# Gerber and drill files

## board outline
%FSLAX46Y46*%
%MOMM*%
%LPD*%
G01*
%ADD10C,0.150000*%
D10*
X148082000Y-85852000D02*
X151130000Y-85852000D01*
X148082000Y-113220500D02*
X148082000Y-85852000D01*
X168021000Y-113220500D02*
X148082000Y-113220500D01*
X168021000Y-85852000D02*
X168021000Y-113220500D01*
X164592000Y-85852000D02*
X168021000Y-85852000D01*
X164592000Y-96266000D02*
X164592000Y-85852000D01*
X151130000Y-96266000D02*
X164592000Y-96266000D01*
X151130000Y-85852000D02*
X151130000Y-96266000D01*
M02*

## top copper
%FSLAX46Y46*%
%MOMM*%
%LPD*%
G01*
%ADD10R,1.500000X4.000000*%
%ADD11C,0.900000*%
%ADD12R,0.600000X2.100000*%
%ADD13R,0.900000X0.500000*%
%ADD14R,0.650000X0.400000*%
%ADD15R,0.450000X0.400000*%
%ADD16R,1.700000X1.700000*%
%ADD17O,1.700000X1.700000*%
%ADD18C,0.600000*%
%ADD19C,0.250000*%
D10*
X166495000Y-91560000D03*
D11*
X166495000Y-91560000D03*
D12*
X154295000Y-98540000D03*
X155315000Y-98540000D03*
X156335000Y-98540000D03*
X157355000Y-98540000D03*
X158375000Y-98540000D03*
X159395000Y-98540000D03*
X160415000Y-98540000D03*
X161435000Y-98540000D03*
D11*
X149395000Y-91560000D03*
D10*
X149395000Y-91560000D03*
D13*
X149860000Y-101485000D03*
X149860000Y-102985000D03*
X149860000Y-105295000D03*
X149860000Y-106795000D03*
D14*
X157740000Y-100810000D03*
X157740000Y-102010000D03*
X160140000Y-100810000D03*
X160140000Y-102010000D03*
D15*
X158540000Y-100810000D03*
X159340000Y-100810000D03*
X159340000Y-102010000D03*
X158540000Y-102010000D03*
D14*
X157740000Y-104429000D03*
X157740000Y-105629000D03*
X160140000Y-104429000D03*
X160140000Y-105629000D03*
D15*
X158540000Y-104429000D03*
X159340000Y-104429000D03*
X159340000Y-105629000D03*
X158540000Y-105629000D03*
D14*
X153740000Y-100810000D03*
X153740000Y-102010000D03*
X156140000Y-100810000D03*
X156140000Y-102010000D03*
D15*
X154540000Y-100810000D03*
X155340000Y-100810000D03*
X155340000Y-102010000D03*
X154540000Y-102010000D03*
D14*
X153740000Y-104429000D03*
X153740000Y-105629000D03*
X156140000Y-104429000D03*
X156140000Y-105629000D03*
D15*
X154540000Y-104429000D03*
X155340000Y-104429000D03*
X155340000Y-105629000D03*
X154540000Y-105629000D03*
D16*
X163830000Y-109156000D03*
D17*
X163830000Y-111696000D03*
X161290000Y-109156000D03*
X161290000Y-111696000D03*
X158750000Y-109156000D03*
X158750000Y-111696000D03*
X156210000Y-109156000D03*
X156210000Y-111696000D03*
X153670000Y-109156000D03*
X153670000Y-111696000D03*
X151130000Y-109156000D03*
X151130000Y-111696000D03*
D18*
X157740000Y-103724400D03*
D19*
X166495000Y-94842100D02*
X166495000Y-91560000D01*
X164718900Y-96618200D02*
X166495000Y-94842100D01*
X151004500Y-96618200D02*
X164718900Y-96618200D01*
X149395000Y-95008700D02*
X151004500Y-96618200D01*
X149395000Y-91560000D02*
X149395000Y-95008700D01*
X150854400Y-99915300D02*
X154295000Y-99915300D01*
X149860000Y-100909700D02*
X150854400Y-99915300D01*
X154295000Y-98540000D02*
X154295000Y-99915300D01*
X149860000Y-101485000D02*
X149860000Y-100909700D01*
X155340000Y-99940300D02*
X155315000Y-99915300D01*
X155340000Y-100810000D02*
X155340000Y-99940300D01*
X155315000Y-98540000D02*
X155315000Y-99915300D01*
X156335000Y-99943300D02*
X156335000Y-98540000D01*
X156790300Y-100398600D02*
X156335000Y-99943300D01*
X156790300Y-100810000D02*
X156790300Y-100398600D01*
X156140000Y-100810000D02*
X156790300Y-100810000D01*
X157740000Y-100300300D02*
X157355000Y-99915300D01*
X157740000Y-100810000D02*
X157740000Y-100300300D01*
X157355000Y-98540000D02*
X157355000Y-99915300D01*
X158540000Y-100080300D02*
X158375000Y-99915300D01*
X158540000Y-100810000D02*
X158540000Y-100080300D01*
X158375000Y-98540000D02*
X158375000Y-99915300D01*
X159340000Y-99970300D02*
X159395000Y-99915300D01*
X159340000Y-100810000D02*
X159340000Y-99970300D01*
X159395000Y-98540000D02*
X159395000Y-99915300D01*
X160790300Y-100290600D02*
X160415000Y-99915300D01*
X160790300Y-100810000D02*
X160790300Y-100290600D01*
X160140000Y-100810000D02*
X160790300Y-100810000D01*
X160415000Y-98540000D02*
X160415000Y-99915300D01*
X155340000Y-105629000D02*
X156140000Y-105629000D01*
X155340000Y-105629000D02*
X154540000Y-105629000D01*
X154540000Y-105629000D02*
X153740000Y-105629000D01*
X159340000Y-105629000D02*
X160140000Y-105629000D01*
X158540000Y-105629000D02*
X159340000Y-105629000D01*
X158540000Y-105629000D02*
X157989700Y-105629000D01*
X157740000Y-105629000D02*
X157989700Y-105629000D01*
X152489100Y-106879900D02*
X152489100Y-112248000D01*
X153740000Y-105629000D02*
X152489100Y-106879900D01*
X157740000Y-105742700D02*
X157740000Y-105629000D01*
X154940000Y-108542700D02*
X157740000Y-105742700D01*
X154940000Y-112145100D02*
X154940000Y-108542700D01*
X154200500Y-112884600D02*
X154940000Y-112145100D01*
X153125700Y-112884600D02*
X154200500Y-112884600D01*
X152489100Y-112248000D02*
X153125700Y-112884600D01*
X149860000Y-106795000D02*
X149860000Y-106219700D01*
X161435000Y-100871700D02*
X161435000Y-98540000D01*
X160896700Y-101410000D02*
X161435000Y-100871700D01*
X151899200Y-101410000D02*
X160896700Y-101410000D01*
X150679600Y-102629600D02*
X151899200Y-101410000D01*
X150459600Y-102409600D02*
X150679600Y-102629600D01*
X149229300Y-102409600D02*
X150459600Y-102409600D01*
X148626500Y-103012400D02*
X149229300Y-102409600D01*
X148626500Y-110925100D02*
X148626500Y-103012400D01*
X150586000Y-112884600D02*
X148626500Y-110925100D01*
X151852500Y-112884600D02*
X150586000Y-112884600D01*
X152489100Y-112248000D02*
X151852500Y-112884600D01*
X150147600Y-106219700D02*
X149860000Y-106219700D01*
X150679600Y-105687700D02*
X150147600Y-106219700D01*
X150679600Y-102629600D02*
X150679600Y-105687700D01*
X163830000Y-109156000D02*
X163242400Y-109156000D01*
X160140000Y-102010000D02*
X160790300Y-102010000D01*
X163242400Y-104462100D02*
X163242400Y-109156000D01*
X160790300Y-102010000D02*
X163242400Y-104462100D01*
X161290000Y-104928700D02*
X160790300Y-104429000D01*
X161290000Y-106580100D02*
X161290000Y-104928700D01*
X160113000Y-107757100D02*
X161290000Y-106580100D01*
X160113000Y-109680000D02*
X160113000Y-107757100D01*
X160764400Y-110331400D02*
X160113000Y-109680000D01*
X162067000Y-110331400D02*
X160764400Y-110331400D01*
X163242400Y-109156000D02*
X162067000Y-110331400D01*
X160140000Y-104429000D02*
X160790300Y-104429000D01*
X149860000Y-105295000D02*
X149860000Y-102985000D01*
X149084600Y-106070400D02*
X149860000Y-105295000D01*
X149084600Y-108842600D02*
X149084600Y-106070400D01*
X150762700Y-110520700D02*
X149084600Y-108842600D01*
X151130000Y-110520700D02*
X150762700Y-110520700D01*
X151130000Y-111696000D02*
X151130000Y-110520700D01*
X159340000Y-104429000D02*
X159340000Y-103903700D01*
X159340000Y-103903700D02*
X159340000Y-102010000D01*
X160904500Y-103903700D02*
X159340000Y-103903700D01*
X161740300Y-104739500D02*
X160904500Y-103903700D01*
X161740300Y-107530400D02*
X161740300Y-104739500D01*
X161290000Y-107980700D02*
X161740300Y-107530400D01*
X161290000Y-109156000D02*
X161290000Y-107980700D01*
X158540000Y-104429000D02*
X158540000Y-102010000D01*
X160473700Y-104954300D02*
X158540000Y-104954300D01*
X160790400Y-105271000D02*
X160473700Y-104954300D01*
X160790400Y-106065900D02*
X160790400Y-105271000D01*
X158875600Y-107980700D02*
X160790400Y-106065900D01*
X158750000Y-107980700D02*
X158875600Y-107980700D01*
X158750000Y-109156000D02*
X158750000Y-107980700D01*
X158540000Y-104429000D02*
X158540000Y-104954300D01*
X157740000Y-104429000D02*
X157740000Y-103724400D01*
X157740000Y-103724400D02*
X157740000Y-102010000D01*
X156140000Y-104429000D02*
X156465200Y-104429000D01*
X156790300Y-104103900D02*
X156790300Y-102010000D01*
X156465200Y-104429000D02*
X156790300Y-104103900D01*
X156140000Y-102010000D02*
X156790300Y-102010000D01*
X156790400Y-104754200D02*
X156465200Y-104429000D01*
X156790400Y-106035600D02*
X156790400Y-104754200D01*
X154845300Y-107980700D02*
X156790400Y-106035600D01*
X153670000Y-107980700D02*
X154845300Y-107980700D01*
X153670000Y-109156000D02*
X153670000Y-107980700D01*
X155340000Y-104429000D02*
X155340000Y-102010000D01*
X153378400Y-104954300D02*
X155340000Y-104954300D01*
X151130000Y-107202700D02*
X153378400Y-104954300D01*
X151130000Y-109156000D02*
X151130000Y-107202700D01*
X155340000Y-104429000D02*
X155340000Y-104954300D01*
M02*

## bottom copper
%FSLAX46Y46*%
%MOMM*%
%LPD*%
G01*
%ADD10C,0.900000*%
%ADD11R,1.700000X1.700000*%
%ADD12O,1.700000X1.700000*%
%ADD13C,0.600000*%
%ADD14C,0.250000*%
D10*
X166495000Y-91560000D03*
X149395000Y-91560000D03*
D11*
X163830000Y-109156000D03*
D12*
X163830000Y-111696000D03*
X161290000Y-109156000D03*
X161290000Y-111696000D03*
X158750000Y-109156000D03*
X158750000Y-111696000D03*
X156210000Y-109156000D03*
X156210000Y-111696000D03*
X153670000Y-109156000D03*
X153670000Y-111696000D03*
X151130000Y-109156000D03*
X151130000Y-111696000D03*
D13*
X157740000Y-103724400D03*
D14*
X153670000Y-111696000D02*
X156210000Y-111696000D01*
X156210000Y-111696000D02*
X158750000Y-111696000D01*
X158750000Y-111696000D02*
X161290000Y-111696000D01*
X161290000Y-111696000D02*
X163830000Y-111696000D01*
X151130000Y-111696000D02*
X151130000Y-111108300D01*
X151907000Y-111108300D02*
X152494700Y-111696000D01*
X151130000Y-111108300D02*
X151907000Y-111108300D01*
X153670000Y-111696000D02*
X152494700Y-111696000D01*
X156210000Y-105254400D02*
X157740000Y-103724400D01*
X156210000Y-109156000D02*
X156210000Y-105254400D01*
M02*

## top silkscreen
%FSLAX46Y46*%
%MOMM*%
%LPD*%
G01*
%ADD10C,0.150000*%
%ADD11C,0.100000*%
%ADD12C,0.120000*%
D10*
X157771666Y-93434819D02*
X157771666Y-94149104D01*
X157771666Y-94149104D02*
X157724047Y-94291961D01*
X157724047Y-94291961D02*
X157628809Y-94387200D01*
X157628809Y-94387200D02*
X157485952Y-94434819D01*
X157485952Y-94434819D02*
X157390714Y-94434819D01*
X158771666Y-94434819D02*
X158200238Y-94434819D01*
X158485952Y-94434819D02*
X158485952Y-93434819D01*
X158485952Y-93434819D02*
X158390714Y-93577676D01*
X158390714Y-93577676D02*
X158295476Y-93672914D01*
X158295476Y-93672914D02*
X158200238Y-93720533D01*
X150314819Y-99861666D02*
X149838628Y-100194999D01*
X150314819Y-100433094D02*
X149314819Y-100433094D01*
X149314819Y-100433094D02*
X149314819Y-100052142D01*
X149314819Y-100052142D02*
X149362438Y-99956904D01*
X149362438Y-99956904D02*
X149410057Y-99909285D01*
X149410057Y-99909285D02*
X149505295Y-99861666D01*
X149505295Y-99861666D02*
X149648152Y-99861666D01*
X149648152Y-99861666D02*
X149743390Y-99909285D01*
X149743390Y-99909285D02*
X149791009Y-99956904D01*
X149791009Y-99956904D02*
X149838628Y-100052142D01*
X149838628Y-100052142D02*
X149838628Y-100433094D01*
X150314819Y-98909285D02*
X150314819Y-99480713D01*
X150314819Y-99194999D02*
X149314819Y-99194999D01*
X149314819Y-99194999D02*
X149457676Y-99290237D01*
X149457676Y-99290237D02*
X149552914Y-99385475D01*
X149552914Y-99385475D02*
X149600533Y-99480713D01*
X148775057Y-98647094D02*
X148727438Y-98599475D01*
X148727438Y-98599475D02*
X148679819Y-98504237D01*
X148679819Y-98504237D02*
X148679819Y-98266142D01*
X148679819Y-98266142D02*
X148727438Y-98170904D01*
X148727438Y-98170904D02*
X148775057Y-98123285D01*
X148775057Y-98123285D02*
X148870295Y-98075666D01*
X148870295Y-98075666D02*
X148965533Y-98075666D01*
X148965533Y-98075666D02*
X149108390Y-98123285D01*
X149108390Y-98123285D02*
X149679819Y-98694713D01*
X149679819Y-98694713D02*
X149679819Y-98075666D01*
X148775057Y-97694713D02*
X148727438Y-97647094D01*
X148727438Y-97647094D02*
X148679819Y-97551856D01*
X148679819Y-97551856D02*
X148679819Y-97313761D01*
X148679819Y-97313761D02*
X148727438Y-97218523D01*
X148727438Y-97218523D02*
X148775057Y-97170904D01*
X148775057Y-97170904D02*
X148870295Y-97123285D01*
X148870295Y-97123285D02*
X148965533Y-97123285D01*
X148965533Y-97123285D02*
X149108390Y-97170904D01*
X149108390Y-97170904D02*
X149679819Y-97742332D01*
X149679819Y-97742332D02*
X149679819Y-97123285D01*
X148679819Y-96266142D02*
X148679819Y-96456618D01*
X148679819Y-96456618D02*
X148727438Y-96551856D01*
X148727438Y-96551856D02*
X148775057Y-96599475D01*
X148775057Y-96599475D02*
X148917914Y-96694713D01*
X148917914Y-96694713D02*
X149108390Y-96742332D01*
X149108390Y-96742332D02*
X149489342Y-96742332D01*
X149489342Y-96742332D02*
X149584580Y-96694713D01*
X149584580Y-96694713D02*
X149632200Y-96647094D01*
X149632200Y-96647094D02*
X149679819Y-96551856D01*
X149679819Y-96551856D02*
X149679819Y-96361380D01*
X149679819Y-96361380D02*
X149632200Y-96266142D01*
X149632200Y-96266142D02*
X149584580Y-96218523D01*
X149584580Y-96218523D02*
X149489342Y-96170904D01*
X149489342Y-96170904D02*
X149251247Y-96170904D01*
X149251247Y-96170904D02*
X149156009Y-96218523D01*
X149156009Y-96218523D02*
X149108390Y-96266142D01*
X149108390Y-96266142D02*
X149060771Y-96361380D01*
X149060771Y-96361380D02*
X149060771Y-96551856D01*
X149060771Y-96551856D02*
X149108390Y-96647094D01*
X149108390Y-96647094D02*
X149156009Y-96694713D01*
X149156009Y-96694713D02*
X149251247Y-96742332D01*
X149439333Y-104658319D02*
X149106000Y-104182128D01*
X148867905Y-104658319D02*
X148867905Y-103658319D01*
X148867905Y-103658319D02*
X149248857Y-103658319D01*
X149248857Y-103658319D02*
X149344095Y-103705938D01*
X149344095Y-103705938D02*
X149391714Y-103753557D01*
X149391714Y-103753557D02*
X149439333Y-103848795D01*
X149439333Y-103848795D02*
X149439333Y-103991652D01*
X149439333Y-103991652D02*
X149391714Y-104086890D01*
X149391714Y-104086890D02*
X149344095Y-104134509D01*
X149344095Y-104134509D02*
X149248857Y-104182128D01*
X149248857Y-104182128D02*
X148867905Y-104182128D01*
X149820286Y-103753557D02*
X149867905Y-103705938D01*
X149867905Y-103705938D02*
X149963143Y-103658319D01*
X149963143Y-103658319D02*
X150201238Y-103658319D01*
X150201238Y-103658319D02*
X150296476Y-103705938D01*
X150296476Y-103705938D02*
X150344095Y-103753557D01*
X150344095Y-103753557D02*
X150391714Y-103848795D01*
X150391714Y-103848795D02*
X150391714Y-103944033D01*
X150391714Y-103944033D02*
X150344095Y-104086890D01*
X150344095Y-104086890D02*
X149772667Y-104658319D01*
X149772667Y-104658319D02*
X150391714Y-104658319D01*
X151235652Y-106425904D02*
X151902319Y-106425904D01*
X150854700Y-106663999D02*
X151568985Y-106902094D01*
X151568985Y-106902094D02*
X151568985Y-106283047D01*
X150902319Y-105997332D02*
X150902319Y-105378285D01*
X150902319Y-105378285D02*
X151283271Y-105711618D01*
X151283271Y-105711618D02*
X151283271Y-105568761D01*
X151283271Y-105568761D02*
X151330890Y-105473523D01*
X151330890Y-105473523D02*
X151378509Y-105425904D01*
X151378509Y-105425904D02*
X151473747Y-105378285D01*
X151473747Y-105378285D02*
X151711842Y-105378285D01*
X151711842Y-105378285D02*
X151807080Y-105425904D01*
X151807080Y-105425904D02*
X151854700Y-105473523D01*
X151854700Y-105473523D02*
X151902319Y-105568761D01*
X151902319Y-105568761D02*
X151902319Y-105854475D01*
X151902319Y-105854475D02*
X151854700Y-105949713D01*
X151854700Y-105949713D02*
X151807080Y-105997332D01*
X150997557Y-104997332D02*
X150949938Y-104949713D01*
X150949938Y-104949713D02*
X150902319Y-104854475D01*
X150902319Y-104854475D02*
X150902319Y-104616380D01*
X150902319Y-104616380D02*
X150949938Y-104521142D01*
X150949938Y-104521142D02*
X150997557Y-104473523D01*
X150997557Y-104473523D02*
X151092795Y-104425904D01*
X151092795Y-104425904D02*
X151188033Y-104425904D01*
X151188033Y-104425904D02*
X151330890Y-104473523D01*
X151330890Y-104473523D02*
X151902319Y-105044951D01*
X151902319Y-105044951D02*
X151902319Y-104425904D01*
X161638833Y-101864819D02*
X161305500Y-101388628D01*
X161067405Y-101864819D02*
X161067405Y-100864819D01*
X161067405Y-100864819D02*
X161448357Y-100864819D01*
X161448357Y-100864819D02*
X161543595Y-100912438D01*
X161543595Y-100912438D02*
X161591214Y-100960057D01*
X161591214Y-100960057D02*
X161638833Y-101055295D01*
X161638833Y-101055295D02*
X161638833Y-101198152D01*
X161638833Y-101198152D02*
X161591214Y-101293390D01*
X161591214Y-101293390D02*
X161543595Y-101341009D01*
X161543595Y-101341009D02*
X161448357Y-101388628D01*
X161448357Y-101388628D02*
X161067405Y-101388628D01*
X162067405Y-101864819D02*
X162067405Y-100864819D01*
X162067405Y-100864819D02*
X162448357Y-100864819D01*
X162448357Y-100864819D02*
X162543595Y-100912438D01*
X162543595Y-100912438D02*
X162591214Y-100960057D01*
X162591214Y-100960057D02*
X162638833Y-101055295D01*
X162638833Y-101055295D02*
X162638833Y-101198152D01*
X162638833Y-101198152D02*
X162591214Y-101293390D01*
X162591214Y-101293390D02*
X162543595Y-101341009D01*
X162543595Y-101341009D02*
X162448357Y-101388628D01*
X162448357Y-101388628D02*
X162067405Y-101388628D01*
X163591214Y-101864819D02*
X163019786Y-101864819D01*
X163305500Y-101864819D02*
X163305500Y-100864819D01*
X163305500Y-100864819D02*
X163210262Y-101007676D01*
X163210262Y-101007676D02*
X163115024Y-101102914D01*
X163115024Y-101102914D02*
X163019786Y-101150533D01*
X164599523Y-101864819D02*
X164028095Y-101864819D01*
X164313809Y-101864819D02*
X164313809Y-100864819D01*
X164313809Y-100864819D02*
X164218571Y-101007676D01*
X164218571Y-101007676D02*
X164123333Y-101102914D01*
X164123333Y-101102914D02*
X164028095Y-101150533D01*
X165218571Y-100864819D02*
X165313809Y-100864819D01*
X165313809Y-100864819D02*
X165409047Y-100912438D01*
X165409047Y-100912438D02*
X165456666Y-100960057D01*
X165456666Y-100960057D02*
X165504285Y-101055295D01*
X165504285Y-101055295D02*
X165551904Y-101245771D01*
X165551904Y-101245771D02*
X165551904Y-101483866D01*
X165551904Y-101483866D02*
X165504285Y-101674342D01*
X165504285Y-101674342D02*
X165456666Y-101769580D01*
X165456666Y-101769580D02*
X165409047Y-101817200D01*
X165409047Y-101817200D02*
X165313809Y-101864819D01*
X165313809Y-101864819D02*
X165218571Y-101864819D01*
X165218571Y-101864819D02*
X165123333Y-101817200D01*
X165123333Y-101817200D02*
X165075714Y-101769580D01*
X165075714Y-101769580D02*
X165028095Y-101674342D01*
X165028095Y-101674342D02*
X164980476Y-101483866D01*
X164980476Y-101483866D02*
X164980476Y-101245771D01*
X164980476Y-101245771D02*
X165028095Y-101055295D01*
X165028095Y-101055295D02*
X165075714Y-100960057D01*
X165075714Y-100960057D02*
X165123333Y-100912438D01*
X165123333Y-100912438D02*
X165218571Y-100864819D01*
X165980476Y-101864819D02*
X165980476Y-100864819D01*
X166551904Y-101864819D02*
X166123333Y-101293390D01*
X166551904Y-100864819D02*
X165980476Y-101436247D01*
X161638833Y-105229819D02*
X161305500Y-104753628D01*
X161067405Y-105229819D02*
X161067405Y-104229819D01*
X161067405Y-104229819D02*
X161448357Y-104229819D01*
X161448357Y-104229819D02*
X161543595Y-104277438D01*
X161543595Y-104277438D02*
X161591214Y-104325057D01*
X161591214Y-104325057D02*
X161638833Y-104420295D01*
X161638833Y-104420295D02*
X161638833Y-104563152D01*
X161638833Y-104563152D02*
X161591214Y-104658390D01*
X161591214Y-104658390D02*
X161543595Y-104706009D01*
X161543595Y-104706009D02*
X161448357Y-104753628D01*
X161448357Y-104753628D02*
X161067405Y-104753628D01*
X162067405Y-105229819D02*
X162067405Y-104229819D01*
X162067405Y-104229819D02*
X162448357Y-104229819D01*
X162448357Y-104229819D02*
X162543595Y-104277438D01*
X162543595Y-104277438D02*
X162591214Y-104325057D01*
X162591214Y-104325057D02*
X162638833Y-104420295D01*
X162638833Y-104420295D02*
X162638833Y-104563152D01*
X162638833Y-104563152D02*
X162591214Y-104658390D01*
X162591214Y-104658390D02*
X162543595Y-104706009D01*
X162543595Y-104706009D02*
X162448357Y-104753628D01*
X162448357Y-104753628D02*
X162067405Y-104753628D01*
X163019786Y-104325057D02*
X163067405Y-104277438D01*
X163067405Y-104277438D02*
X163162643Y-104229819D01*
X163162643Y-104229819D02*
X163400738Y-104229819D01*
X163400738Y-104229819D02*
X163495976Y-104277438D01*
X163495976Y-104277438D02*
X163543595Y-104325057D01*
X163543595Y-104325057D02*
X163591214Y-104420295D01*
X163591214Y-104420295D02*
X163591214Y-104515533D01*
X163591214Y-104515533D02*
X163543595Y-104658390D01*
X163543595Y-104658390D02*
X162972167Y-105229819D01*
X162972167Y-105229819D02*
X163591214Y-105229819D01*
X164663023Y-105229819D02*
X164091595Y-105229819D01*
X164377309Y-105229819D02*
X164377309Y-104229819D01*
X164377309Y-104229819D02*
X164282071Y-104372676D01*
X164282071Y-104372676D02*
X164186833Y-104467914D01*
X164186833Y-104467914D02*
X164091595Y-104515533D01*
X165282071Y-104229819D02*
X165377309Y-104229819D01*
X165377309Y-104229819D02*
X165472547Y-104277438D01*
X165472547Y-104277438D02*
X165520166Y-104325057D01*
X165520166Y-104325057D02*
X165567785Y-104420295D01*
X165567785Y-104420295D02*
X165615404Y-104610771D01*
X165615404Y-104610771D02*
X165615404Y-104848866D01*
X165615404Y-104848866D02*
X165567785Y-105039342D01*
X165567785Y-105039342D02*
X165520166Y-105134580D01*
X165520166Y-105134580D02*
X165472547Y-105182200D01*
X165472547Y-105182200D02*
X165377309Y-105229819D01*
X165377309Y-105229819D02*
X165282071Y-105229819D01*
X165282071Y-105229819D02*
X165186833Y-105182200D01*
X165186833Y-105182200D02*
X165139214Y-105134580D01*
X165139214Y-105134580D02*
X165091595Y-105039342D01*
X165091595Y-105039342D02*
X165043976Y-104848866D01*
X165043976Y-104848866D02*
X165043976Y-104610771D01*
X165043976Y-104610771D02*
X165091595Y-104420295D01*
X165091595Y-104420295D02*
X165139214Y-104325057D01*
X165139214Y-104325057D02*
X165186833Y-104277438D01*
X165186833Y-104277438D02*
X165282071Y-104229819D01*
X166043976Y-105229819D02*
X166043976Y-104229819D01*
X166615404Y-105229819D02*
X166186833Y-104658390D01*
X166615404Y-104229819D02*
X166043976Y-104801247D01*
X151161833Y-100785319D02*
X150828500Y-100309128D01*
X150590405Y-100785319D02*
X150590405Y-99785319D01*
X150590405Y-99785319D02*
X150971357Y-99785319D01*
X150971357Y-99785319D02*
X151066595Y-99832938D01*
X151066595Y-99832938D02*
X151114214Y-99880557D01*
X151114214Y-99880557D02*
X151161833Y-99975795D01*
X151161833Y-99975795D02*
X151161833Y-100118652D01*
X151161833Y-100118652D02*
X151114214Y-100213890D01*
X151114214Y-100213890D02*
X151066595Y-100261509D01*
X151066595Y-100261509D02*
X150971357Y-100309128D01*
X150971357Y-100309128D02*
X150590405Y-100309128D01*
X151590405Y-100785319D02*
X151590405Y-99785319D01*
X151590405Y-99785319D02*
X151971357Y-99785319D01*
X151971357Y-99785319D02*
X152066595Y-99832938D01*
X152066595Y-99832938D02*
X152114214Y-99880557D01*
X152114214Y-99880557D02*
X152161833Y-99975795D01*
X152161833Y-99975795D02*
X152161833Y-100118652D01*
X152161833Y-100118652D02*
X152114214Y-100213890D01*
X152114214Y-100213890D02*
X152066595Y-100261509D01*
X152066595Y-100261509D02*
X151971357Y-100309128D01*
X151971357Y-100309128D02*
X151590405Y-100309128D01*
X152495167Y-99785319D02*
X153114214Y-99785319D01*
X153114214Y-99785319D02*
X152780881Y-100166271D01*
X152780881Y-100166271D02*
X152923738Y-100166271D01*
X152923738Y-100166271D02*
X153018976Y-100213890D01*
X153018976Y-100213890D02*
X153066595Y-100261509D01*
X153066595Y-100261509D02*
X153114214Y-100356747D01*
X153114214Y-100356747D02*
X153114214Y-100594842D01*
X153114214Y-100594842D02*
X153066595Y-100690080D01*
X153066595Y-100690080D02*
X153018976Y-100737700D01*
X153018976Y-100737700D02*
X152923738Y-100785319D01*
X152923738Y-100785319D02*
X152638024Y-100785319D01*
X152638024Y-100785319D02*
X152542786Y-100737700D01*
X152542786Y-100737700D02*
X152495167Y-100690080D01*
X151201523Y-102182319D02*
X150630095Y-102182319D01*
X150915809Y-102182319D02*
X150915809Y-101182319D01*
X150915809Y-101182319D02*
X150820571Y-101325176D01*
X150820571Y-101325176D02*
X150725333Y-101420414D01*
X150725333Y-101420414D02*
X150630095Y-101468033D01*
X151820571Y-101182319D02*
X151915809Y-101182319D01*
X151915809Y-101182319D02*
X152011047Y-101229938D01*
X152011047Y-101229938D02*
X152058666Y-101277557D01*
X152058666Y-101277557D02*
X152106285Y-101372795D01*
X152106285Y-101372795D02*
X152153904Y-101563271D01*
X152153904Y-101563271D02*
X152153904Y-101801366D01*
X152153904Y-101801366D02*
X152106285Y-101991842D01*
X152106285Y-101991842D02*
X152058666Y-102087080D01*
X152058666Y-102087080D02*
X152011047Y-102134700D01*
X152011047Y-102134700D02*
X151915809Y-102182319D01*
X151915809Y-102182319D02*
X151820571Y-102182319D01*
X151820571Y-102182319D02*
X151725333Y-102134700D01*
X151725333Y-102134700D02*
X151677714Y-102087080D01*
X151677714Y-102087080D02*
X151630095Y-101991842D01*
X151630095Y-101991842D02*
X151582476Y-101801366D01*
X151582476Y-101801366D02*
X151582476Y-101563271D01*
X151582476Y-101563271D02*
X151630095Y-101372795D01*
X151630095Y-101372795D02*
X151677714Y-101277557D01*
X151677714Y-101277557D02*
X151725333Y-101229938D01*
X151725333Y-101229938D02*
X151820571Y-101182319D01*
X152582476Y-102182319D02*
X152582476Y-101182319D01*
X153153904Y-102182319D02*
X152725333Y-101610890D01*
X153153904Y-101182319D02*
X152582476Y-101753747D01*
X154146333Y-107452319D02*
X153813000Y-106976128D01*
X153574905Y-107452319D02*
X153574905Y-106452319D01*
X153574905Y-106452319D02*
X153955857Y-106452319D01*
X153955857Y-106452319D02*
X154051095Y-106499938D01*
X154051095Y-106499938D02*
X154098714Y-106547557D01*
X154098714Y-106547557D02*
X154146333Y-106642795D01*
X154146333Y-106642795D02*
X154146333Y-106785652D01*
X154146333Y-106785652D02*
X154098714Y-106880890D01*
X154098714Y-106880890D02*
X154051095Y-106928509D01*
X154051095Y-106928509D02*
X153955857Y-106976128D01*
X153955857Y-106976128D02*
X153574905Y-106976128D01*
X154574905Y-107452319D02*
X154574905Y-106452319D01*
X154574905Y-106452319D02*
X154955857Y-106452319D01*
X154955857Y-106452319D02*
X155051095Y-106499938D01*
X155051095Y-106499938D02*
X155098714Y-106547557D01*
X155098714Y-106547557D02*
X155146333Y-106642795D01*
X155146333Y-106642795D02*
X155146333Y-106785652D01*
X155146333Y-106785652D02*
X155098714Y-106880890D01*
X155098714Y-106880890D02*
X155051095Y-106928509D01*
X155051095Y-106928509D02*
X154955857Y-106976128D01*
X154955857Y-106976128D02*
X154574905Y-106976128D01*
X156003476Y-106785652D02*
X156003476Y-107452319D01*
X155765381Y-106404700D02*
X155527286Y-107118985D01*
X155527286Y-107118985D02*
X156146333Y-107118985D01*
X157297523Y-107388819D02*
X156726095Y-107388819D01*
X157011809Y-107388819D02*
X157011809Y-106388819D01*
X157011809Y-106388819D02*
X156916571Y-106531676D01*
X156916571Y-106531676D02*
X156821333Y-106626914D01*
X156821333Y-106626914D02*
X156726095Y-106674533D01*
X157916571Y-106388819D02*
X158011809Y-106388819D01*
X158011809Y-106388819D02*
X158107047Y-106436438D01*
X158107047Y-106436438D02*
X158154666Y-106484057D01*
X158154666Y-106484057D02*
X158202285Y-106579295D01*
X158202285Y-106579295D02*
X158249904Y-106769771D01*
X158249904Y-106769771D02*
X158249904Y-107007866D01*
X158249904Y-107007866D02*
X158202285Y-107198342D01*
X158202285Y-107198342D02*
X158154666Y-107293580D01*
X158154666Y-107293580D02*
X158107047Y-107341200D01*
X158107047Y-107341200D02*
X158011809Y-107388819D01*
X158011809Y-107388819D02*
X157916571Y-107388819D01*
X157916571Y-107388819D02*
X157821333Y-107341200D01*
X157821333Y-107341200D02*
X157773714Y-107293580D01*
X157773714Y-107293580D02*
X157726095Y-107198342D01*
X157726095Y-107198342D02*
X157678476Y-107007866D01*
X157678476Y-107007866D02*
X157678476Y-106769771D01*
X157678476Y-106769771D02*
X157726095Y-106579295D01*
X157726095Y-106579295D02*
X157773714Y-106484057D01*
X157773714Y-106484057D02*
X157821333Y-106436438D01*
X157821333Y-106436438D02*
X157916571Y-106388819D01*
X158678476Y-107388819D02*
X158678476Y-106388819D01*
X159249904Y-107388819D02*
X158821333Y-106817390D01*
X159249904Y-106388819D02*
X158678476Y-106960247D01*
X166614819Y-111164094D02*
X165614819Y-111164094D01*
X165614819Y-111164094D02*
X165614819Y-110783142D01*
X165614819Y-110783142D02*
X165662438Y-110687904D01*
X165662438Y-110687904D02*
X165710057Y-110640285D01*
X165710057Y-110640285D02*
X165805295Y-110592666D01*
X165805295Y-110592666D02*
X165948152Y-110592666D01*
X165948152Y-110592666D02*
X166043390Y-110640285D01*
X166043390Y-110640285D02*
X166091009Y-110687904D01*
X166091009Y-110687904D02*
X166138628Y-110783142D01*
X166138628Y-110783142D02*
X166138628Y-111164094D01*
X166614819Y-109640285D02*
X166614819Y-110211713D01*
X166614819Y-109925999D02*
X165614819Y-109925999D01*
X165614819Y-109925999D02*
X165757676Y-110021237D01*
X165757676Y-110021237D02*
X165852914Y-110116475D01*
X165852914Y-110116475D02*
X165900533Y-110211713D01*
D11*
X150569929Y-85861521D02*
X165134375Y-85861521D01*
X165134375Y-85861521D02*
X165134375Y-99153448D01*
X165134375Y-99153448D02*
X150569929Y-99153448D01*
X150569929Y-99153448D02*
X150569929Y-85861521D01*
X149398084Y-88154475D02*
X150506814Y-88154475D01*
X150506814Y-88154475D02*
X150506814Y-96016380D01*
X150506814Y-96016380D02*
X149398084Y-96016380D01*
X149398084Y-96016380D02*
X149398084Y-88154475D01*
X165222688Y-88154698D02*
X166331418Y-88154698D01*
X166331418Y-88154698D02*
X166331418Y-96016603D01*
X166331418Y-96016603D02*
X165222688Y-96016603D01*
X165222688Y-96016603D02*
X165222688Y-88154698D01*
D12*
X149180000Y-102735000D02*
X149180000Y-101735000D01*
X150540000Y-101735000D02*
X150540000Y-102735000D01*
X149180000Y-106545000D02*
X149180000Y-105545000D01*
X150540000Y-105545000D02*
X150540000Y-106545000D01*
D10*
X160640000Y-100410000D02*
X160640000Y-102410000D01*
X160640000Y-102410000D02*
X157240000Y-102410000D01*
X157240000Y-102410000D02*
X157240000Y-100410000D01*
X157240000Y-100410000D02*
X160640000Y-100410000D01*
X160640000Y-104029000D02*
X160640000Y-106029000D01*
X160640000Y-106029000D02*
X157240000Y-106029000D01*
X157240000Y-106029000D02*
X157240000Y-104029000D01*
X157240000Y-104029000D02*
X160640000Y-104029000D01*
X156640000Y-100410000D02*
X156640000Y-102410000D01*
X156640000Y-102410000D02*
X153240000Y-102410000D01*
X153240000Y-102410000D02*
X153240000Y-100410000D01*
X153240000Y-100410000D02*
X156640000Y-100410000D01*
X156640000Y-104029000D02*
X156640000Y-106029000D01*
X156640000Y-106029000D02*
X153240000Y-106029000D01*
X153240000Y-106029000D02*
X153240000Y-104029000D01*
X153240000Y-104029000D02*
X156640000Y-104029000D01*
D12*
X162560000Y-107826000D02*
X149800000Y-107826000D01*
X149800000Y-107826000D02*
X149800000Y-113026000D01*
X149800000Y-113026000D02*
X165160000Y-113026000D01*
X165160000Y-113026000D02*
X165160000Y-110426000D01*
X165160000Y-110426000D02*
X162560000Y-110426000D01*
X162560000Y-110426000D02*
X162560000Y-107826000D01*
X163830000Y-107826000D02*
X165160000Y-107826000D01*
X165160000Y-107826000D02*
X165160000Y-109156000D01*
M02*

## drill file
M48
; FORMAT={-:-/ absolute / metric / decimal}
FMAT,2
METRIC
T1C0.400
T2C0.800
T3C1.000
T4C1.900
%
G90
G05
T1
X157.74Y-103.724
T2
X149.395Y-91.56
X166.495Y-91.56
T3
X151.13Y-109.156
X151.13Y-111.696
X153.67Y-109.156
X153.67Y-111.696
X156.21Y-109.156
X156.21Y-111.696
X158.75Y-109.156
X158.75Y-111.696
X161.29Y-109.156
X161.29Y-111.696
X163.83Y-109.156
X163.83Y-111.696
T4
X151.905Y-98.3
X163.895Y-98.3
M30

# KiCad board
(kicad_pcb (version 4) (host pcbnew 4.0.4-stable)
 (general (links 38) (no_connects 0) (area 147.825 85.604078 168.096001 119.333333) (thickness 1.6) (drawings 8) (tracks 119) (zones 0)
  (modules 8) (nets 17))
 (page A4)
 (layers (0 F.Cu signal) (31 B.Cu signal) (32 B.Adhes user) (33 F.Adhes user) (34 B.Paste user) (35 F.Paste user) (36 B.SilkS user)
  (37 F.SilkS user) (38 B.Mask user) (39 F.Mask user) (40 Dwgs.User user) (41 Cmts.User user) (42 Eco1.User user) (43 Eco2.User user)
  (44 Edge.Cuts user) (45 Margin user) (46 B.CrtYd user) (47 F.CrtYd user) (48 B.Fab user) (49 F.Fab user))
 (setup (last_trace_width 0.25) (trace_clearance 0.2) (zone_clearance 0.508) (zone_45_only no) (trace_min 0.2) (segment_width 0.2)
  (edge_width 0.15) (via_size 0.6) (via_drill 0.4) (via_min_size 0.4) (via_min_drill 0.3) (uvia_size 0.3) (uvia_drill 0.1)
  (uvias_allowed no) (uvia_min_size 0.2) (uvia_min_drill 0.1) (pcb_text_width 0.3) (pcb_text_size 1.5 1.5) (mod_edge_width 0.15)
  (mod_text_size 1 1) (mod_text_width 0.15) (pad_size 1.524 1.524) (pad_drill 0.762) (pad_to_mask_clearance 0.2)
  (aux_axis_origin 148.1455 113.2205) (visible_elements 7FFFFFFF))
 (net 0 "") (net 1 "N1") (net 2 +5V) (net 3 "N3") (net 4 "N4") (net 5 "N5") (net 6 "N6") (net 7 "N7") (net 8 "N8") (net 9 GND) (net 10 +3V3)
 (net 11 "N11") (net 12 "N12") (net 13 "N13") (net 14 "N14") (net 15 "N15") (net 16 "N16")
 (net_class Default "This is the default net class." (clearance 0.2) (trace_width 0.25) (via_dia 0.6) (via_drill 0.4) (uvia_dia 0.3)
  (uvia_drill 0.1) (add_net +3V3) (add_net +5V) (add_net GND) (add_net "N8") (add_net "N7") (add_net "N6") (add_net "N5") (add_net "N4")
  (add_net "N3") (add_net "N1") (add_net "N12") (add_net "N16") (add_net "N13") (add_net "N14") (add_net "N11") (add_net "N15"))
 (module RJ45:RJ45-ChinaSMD (layer F.Cu) (at 150.495 99.06)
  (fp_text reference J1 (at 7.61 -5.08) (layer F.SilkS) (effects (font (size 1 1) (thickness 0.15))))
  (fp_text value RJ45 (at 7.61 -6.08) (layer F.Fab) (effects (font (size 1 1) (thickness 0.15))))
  (fp_line (start 0.074929 -13.198479) (end 14.639375 -13.198479) (layer F.SilkS) (width 0.1))
  (fp_line (start 14.639375 -13.198479) (end 14.639375 0.093448) (layer F.SilkS) (width 0.1))
  (fp_line (start 14.639375 0.093448) (end 0.074929 0.093448) (layer F.SilkS) (width 0.1))
  (fp_line (start 0.074929 0.093448) (end 0.074929 -13.198479) (layer F.SilkS) (width 0.1))
  (fp_line (start -1.096916 -10.905525) (end 0.011814 -10.905525) (layer F.SilkS) (width 0.1))
  (fp_line (start 0.011814 -10.905525) (end 0.011814 -3.04362) (layer F.SilkS) (width 0.1))
  (fp_line (start 0.011814 -3.04362) (end -1.096916 -3.04362) (layer F.SilkS) (width 0.1))
  (fp_line (start -1.096916 -3.04362) (end -1.096916 -10.905525) (layer F.SilkS) (width 0.1))
  (fp_line (start 14.727688 -10.905302) (end 15.836418 -10.905302) (layer F.SilkS) (width 0.1))
  (fp_line (start 15.836418 -10.905302) (end 15.836418 -3.043397) (layer F.SilkS) (width 0.1))
  (fp_line (start 15.836418 -3.043397) (end 14.727688 -3.043397) (layer F.SilkS) (width 0.1))
  (fp_line (start 14.727688 -3.043397) (end 14.727688 -10.905302) (layer F.SilkS) (width 0.1))
  (pad 9 smd rect (at 16 -7.5) (size 1.5 4) (layers F.Cu F.Paste F.Mask) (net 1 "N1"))
  (pad 9 thru_hole circle (at 16 -7.5) (size 0.9 0.9) (drill 0.8) (layers *.Cu *.Mask) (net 1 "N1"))
  (pad "" np_thru_hole circle (at 13.4 -0.76) (size 1.9 1.9) (drill 1.9) (layers *.Cu *.Mask))
  (pad "" np_thru_hole circle (at 1.41 -0.76) (size 1.9 1.9) (drill 1.9) (layers *.Cu *.Mask))
  (pad 8 smd rect (at 3.8 -0.52) (size 0.6 2.1) (layers F.Cu F.Paste F.Mask) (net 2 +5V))
  (pad 7 smd rect (at 4.82 -0.52) (size 0.6 2.1) (layers F.Cu F.Paste F.Mask) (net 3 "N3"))
  (pad 6 smd rect (at 5.84 -0.52) (size 0.6 2.1) (layers F.Cu F.Paste F.Mask) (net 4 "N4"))
  (pad 5 smd rect (at 6.86 -0.52) (size 0.6 2.1) (layers F.Cu F.Paste F.Mask) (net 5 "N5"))
  (pad 4 smd rect (at 7.88 -0.52) (size 0.6 2.1) (layers F.Cu F.Paste F.Mask) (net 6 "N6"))
  (pad 3 smd rect (at 8.9 -0.52) (size 0.6 2.1) (layers F.Cu F.Paste F.Mask) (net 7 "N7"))
  (pad 2 smd rect (at 9.92 -0.52) (size 0.6 2.1) (layers F.Cu F.Paste F.Mask) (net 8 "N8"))
  (pad 1 smd rect (at 10.94 -0.52) (size 0.6 2.1) (layers F.Cu F.Paste F.Mask) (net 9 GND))
  (pad 9 thru_hole circle (at -1.1 -7.5) (size 0.9 0.9) (drill 0.8) (layers *.Cu *.Mask) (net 1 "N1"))
  (pad 9 smd rect (at -1.1 -7.5) (size 1.5 4) (layers F.Cu F.Paste F.Mask) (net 1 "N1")))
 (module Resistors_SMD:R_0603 (layer F.Cu) (at 149.86 102.235 270)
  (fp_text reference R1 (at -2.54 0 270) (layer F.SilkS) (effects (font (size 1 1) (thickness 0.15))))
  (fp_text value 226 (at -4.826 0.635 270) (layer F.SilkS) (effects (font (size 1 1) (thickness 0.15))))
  (fp_line (start 0.5 0.68) (end -0.5 0.68) (layer F.SilkS) (width 0.12))
  (fp_line (start -0.5 -0.68) (end 0.5 -0.68) (layer F.SilkS) (width 0.12))
  (pad 1 smd rect (at -0.75 0 270) (size 0.5 0.9) (layers F.Cu F.Paste F.Mask) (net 2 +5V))
  (pad 2 smd rect (at 0.75 0 270) (size 0.5 0.9) (layers F.Cu F.Paste F.Mask) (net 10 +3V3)))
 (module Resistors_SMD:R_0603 (layer F.Cu) (at 149.86 106.045 270)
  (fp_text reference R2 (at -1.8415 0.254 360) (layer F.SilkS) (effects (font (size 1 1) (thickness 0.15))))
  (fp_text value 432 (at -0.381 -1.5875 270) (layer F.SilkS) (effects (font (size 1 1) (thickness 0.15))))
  (fp_line (start 0.5 0.68) (end -0.5 0.68) (layer F.SilkS) (width 0.12))
  (fp_line (start -0.5 -0.68) (end 0.5 -0.68) (layer F.SilkS) (width 0.12))
  (pad 1 smd rect (at -0.75 0 270) (size 0.5 0.9) (layers F.Cu F.Paste F.Mask) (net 10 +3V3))
  (pad 2 smd rect (at 0.75 0 270) (size 0.5 0.9) (layers F.Cu F.Paste F.Mask) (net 9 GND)))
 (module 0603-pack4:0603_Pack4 (layer F.Cu) (at 158.94 101.41)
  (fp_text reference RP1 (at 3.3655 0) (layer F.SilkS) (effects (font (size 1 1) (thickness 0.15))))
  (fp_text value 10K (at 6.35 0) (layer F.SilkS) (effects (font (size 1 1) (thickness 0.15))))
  (fp_line (start 1.7 -1) (end 1.7 1) (layer F.SilkS) (width 0.15))
  (fp_line (start 1.7 1) (end -1.7 1) (layer F.SilkS) (width 0.15))
  (fp_line (start -1.7 1) (end -1.7 -1) (layer F.SilkS) (width 0.15))
  (fp_line (start -1.7 -1) (end 1.7 -1) (layer F.SilkS) (width 0.15))
  (pad 1 smd rect (at -1.2 -0.6) (size 0.65 0.4) (layers F.Cu F.Paste F.Mask) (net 5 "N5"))
  (pad 8 smd rect (at -1.2 0.6) (size 0.65 0.4) (layers F.Cu F.Paste F.Mask) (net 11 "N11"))
  (pad 4 smd rect (at 1.2 -0.6) (size 0.65 0.4) (layers F.Cu F.Paste F.Mask) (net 8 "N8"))
  (pad 5 smd rect (at 1.2 0.6) (size 0.65 0.4) (layers F.Cu F.Paste F.Mask) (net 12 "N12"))
  (pad 2 smd rect (at -0.4 -0.6) (size 0.45 0.4) (layers F.Cu F.Paste F.Mask) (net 6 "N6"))
  (pad 3 smd rect (at 0.4 -0.6) (size 0.45 0.4) (layers F.Cu F.Paste F.Mask) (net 7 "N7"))
  (pad 6 smd rect (at 0.4 0.6) (size 0.45 0.4) (layers F.Cu F.Paste F.Mask) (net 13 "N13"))
  (pad 7 smd rect (at -0.4 0.6) (size 0.45 0.4) (layers F.Cu F.Paste F.Mask) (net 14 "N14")))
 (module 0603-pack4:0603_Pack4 (layer F.Cu) (at 158.94 105.029)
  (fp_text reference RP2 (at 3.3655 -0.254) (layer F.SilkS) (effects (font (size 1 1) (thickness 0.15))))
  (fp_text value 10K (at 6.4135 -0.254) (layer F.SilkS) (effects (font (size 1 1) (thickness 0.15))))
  (fp_line (start 1.7 -1) (end 1.7 1) (layer F.SilkS) (width 0.15))
  (fp_line (start 1.7 1) (end -1.7 1) (layer F.SilkS) (width 0.15))
  (fp_line (start -1.7 1) (end -1.7 -1) (layer F.SilkS) (width 0.15))
  (fp_line (start -1.7 -1) (end 1.7 -1) (layer F.SilkS) (width 0.15))
  (pad 1 smd rect (at -1.2 -0.6) (size 0.65 0.4) (layers F.Cu F.Paste F.Mask) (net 11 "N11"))
  (pad 8 smd rect (at -1.2 0.6) (size 0.65 0.4) (layers F.Cu F.Paste F.Mask) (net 9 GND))
  (pad 4 smd rect (at 1.2 -0.6) (size 0.65 0.4) (layers F.Cu F.Paste F.Mask) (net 12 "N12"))
  (pad 5 smd rect (at 1.2 0.6) (size 0.65 0.4) (layers F.Cu F.Paste F.Mask) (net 9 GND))
  (pad 2 smd rect (at -0.4 -0.6) (size 0.45 0.4) (layers F.Cu F.Paste F.Mask) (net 14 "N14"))
  (pad 3 smd rect (at 0.4 -0.6) (size 0.45 0.4) (layers F.Cu F.Paste F.Mask) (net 13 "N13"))
  (pad 6 smd rect (at 0.4 0.6) (size 0.45 0.4) (layers F.Cu F.Paste F.Mask) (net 9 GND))
  (pad 7 smd rect (at -0.4 0.6) (size 0.45 0.4) (layers F.Cu F.Paste F.Mask) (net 9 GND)))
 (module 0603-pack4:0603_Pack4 (layer F.Cu) (at 154.94 101.41)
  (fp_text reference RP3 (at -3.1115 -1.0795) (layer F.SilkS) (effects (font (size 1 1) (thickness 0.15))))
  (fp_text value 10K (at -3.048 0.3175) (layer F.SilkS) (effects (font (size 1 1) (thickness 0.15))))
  (fp_line (start 1.7 -1) (end 1.7 1) (layer F.SilkS) (width 0.15))
  (fp_line (start 1.7 1) (end -1.7 1) (layer F.SilkS) (width 0.15))
  (fp_line (start -1.7 1) (end -1.7 -1) (layer F.SilkS) (width 0.15))
  (fp_line (start -1.7 -1) (end 1.7 -1) (layer F.SilkS) (width 0.15))
  (pad 1 smd rect (at -1.2 -0.6) (size 0.65 0.4) (layers F.Cu F.Paste F.Mask))
  (pad 8 smd rect (at -1.2 0.6) (size 0.65 0.4) (layers F.Cu F.Paste F.Mask))
  (pad 4 smd rect (at 1.2 -0.6) (size 0.65 0.4) (layers F.Cu F.Paste F.Mask) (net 4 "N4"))
  (pad 5 smd rect (at 1.2 0.6) (size 0.65 0.4) (layers F.Cu F.Paste F.Mask) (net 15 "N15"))
  (pad 2 smd rect (at -0.4 -0.6) (size 0.45 0.4) (layers F.Cu F.Paste F.Mask))
  (pad 3 smd rect (at 0.4 -0.6) (size 0.45 0.4) (layers F.Cu F.Paste F.Mask) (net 3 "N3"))
  (pad 6 smd rect (at 0.4 0.6) (size 0.45 0.4) (layers F.Cu F.Paste F.Mask) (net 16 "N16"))
  (pad 7 smd rect (at -0.4 0.6) (size 0.45 0.4) (layers F.Cu F.Paste F.Mask)))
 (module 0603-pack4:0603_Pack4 (layer F.Cu) (at 154.94 105.029)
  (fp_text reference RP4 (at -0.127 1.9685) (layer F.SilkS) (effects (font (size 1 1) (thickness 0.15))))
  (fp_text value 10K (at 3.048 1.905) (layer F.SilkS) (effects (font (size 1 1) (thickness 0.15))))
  (fp_line (start 1.7 -1) (end 1.7 1) (layer F.SilkS) (width 0.15))
  (fp_line (start 1.7 1) (end -1.7 1) (layer F.SilkS) (width 0.15))
  (fp_line (start -1.7 1) (end -1.7 -1) (layer F.SilkS) (width 0.15))
  (fp_line (start -1.7 -1) (end 1.7 -1) (layer F.SilkS) (width 0.15))
  (pad 1 smd rect (at -1.2 -0.6) (size 0.65 0.4) (layers F.Cu F.Paste F.Mask))
  (pad 8 smd rect (at -1.2 0.6) (size 0.65 0.4) (layers F.Cu F.Paste F.Mask) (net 9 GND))
  (pad 4 smd rect (at 1.2 -0.6) (size 0.65 0.4) (layers F.Cu F.Paste F.Mask) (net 15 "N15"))
  (pad 5 smd rect (at 1.2 0.6) (size 0.65 0.4) (layers F.Cu F.Paste F.Mask) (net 9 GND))
  (pad 2 smd rect (at -0.4 -0.6) (size 0.45 0.4) (layers F.Cu F.Paste F.Mask))
  (pad 3 smd rect (at 0.4 -0.6) (size 0.45 0.4) (layers F.Cu F.Paste F.Mask) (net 16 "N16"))
  (pad 6 smd rect (at 0.4 0.6) (size 0.45 0.4) (layers F.Cu F.Paste F.Mask) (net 9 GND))
  (pad 7 smd rect (at -0.4 0.6) (size 0.45 0.4) (layers F.Cu F.Paste F.Mask) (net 9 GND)))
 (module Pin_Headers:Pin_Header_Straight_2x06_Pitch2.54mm (layer F.Cu) (at 163.83 109.156 270)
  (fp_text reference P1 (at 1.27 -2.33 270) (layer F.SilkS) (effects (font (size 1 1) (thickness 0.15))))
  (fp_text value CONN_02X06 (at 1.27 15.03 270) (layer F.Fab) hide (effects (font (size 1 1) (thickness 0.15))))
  (fp_line (start -1.33 1.27) (end -1.33 14.03) (layer F.SilkS) (width 0.12))
  (fp_line (start -1.33 14.03) (end 3.87 14.03) (layer F.SilkS) (width 0.12))
  (fp_line (start 3.87 14.03) (end 3.87 -1.33) (layer F.SilkS) (width 0.12))
  (fp_line (start 3.87 -1.33) (end 1.27 -1.33) (layer F.SilkS) (width 0.12))
  (fp_line (start 1.27 -1.33) (end 1.27 1.27) (layer F.SilkS) (width 0.12))
  (fp_line (start 1.27 1.27) (end -1.33 1.27) (layer F.SilkS) (width 0.12))
  (fp_line (start -1.33 0) (end -1.33 -1.33) (layer F.SilkS) (width 0.12))
  (fp_line (start -1.33 -1.33) (end 0 -1.33) (layer F.SilkS) (width 0.12))
  (pad 1 thru_hole rect (at 0 0 270) (size 1.7 1.7) (drill 1) (layers *.Cu *.Mask) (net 12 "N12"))
  (pad 2 thru_hole oval (at 2.54 0 270) (size 1.7 1.7) (drill 1) (layers *.Cu *.Mask) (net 10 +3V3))
  (pad 3 thru_hole oval (at 0 2.54 270) (size 1.7 1.7) (drill 1) (layers *.Cu *.Mask) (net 13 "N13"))
  (pad 4 thru_hole oval (at 2.54 2.54 270) (size 1.7 1.7) (drill 1) (layers *.Cu *.Mask) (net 10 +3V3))
  (pad 5 thru_hole oval (at 0 5.08 270) (size 1.7 1.7) (drill 1) (layers *.Cu *.Mask) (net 14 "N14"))
  (pad 6 thru_hole oval (at 2.54 5.08 270) (size 1.7 1.7) (drill 1) (layers *.Cu *.Mask) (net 10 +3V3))
  (pad 7 thru_hole oval (at 0 7.62 270) (size 1.7 1.7) (drill 1) (layers *.Cu *.Mask) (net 11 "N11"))
  (pad 8 thru_hole oval (at 2.54 7.62 270) (size 1.7 1.7) (drill 1) (layers *.Cu *.Mask) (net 10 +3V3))
  (pad 9 thru_hole oval (at 0 10.16 270) (size 1.7 1.7) (drill 1) (layers *.Cu *.Mask) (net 15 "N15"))
  (pad 10 thru_hole oval (at 2.54 10.16 270) (size 1.7 1.7) (drill 1) (layers *.Cu *.Mask) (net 10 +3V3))
  (pad 11 thru_hole oval (at 0 12.7 270) (size 1.7 1.7) (drill 1) (layers *.Cu *.Mask) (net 16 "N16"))
  (pad 12 thru_hole oval (at 2.54 12.7 270) (size 1.7 1.7) (drill 1) (layers *.Cu *.Mask) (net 10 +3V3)))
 (gr_line (start 148.082 85.852) (end 151.13 85.852) (angle 90) (layer Edge.Cuts) (width 0.15))
 (gr_line (start 148.082 113.2205) (end 148.082 85.852) (angle 90) (layer Edge.Cuts) (width 0.15))
 (gr_line (start 168.021 113.2205) (end 148.082 113.2205) (angle 90) (layer Edge.Cuts) (width 0.15))
 (gr_line (start 168.021 85.852) (end 168.021 113.2205) (angle 90) (layer Edge.Cuts) (width 0.15))
 (gr_line (start 164.592 85.852) (end 168.021 85.852) (angle 90) (layer Edge.Cuts) (width 0.15))
 (gr_line (start 164.592 96.266) (end 164.592 85.852) (angle 90) (layer Edge.Cuts) (width 0.15))
 (gr_line (start 151.13 96.266) (end 164.592 96.266) (angle 90) (layer Edge.Cuts) (width 0.15))
 (gr_line (start 151.13 85.852) (end 151.13 96.266) (angle 90) (layer Edge.Cuts) (width 0.15))
 (segment (start 166.495 94.8421) (end 166.495 91.56) (width 0.25) (layer F.Cu) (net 1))
 (segment (start 164.7189 96.6182) (end 166.495 94.8421) (width 0.25) (layer F.Cu) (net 1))
 (segment (start 151.0045 96.6182) (end 164.7189 96.6182) (width 0.25) (layer F.Cu) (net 1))
 (segment (start 149.395 95.0087) (end 151.0045 96.6182) (width 0.25) (layer F.Cu) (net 1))
 (segment (start 149.395 91.56) (end 149.395 95.0087) (width 0.25) (layer F.Cu) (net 1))
 (segment (start 150.8544 99.9153) (end 154.295 99.9153) (width 0.25) (layer F.Cu) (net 2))
 (segment (start 149.86 100.9097) (end 150.8544 99.9153) (width 0.25) (layer F.Cu) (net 2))
 (segment (start 154.295 98.54) (end 154.295 99.9153) (width 0.25) (layer F.Cu) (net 2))
 (segment (start 149.86 101.485) (end 149.86 100.9097) (width 0.25) (layer F.Cu) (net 2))
 (segment (start 155.34 99.9403) (end 155.315 99.9153) (width 0.25) (layer F.Cu) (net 3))
 (segment (start 155.34 100.81) (end 155.34 99.9403) (width 0.25) (layer F.Cu) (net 3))
 (segment (start 155.315 98.54) (end 155.315 99.9153) (width 0.25) (layer F.Cu) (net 3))
 (segment (start 156.335 99.9433) (end 156.335 98.54) (width 0.25) (layer F.Cu) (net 4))
 (segment (start 156.7903 100.3986) (end 156.335 99.9433) (width 0.25) (layer F.Cu) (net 4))
 (segment (start 156.7903 100.81) (end 156.7903 100.3986) (width 0.25) (layer F.Cu) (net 4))
 (segment (start 156.14 100.81) (end 156.7903 100.81) (width 0.25) (layer F.Cu) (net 4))
 (segment (start 157.74 100.3003) (end 157.355 99.9153) (width 0.25) (layer F.Cu) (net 5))
 (segment (start 157.74 100.81) (end 157.74 100.3003) (width 0.25) (layer F.Cu) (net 5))
 (segment (start 157.355 98.54) (end 157.355 99.9153) (width 0.25) (layer F.Cu) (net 5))
 (segment (start 158.54 100.0803) (end 158.375 99.9153) (width 0.25) (layer F.Cu) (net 6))
 (segment (start 158.54 100.81) (end 158.54 100.0803) (width 0.25) (layer F.Cu) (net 6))
 (segment (start 158.375 98.54) (end 158.375 99.9153) (width 0.25) (layer F.Cu) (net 6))
 (segment (start 159.34 99.9703) (end 159.395 99.9153) (width 0.25) (layer F.Cu) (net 7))
 (segment (start 159.34 100.81) (end 159.34 99.9703) (width 0.25) (layer F.Cu) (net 7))
 (segment (start 159.395 98.54) (end 159.395 99.9153) (width 0.25) (layer F.Cu) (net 7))
 (segment (start 160.7903 100.2906) (end 160.415 99.9153) (width 0.25) (layer F.Cu) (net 8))
 (segment (start 160.7903 100.81) (end 160.7903 100.2906) (width 0.25) (layer F.Cu) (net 8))
 (segment (start 160.14 100.81) (end 160.7903 100.81) (width 0.25) (layer F.Cu) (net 8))
 (segment (start 160.415 98.54) (end 160.415 99.9153) (width 0.25) (layer F.Cu) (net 8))
 (segment (start 155.34 105.629) (end 156.14 105.629) (width 0.25) (layer F.Cu) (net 9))
 (segment (start 155.34 105.629) (end 154.54 105.629) (width 0.25) (layer F.Cu) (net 9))
 (segment (start 154.54 105.629) (end 153.74 105.629) (width 0.25) (layer F.Cu) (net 9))
 (segment (start 159.34 105.629) (end 160.14 105.629) (width 0.25) (layer F.Cu) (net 9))
 (segment (start 158.54 105.629) (end 159.34 105.629) (width 0.25) (layer F.Cu) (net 9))
 (segment (start 158.54 105.629) (end 157.9897 105.629) (width 0.25) (layer F.Cu) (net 9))
 (segment (start 157.74 105.629) (end 157.9897 105.629) (width 0.25) (layer F.Cu) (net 9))
 (segment (start 152.4891 106.8799) (end 152.4891 112.248) (width 0.25) (layer F.Cu) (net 9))
 (segment (start 153.74 105.629) (end 152.4891 106.8799) (width 0.25) (layer F.Cu) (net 9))
 (segment (start 157.74 105.7427) (end 157.74 105.629) (width 0.25) (layer F.Cu) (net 9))
 (segment (start 154.94 108.5427) (end 157.74 105.7427) (width 0.25) (layer F.Cu) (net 9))
 (segment (start 154.94 112.1451) (end 154.94 108.5427) (width 0.25) (layer F.Cu) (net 9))
 (segment (start 154.2005 112.8846) (end 154.94 112.1451) (width 0.25) (layer F.Cu) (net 9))
 (segment (start 153.1257 112.8846) (end 154.2005 112.8846) (width 0.25) (layer F.Cu) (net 9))
 (segment (start 152.4891 112.248) (end 153.1257 112.8846) (width 0.25) (layer F.Cu) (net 9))
 (segment (start 149.86 106.795) (end 149.86 106.2197) (width 0.25) (layer F.Cu) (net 9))
 (segment (start 161.435 100.8717) (end 161.435 98.54) (width 0.25) (layer F.Cu) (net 9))
 (segment (start 160.8967 101.41) (end 161.435 100.8717) (width 0.25) (layer F.Cu) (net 9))
 (segment (start 151.8992 101.41) (end 160.8967 101.41) (width 0.25) (layer F.Cu) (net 9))
 (segment (start 150.6796 102.6296) (end 151.8992 101.41) (width 0.25) (layer F.Cu) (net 9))
 (segment (start 150.4596 102.4096) (end 150.6796 102.6296) (width 0.25) (layer F.Cu) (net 9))
 (segment (start 149.2293 102.4096) (end 150.4596 102.4096) (width 0.25) (layer F.Cu) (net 9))
 (segment (start 148.6265 103.0124) (end 149.2293 102.4096) (width 0.25) (layer F.Cu) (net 9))
 (segment (start 148.6265 110.9251) (end 148.6265 103.0124) (width 0.25) (layer F.Cu) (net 9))
 (segment (start 150.586 112.8846) (end 148.6265 110.9251) (width 0.25) (layer F.Cu) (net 9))
 (segment (start 151.8525 112.8846) (end 150.586 112.8846) (width 0.25) (layer F.Cu) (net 9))
 (segment (start 152.4891 112.248) (end 151.8525 112.8846) (width 0.25) (layer F.Cu) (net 9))
 (segment (start 150.1476 106.2197) (end 149.86 106.2197) (width 0.25) (layer F.Cu) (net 9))
 (segment (start 150.6796 105.6877) (end 150.1476 106.2197) (width 0.25) (layer F.Cu) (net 9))
 (segment (start 150.6796 102.6296) (end 150.6796 105.6877) (width 0.25) (layer F.Cu) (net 9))
 (segment (start 163.83 109.156) (end 163.2424 109.156) (width 0.25) (layer F.Cu) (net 12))
 (segment (start 160.14 102.01) (end 160.7903 102.01) (width 0.25) (layer F.Cu) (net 12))
 (segment (start 163.2424 104.4621) (end 163.2424 109.156) (width 0.25) (layer F.Cu) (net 12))
 (segment (start 160.7903 102.01) (end 163.2424 104.4621) (width 0.25) (layer F.Cu) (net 12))
 (segment (start 161.29 104.9287) (end 160.7903 104.429) (width 0.25) (layer F.Cu) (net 12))
 (segment (start 161.29 106.5801) (end 161.29 104.9287) (width 0.25) (layer F.Cu) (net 12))
 (segment (start 160.113 107.7571) (end 161.29 106.5801) (width 0.25) (layer F.Cu) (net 12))
 (segment (start 160.113 109.68) (end 160.113 107.7571) (width 0.25) (layer F.Cu) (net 12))
 (segment (start 160.7644 110.3314) (end 160.113 109.68) (width 0.25) (layer F.Cu) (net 12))
 (segment (start 162.067 110.3314) (end 160.7644 110.3314) (width 0.25) (layer F.Cu) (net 12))
 (segment (start 163.2424 109.156) (end 162.067 110.3314) (width 0.25) (layer F.Cu) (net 12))
 (segment (start 160.14 104.429) (end 160.7903 104.429) (width 0.25) (layer F.Cu) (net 12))
 (segment (start 153.67 111.696) (end 156.21 111.696) (width 0.25) (layer B.Cu) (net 10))
 (segment (start 156.21 111.696) (end 158.75 111.696) (width 0.25) (layer B.Cu) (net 10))
 (segment (start 158.75 111.696) (end 161.29 111.696) (width 0.25) (layer B.Cu) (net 10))
 (segment (start 161.29 111.696) (end 163.83 111.696) (width 0.25) (layer B.Cu) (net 10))
 (segment (start 151.13 111.696) (end 151.13 111.1083) (width 0.25) (layer B.Cu) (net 10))
 (segment (start 151.907 111.1083) (end 152.4947 111.696) (width 0.25) (layer B.Cu) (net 10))
 (segment (start 151.13 111.1083) (end 151.907 111.1083) (width 0.25) (layer B.Cu) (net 10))
 (segment (start 153.67 111.696) (end 152.4947 111.696) (width 0.25) (layer B.Cu) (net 10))
 (segment (start 149.86 105.295) (end 149.86 102.985) (width 0.25) (layer F.Cu) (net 10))
 (segment (start 149.0846 106.0704) (end 149.86 105.295) (width 0.25) (layer F.Cu) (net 10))
 (segment (start 149.0846 108.8426) (end 149.0846 106.0704) (width 0.25) (layer F.Cu) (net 10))
 (segment (start 150.7627 110.5207) (end 149.0846 108.8426) (width 0.25) (layer F.Cu) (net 10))
 (segment (start 151.13 110.5207) (end 150.7627 110.5207) (width 0.25) (layer F.Cu) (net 10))
 (segment (start 151.13 111.696) (end 151.13 110.5207) (width 0.25) (layer F.Cu) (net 10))
 (segment (start 159.34 104.429) (end 159.34 103.9037) (width 0.25) (layer F.Cu) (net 13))
 (segment (start 159.34 103.9037) (end 159.34 102.01) (width 0.25) (layer F.Cu) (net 13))
 (segment (start 160.9045 103.9037) (end 159.34 103.9037) (width 0.25) (layer F.Cu) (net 13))
 (segment (start 161.7403 104.7395) (end 160.9045 103.9037) (width 0.25) (layer F.Cu) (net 13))
 (segment (start 161.7403 107.5304) (end 161.7403 104.7395) (width 0.25) (layer F.Cu) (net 13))
 (segment (start 161.29 107.9807) (end 161.7403 107.5304) (width 0.25) (layer F.Cu) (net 13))
 (segment (start 161.29 109.156) (end 161.29 107.9807) (width 0.25) (layer F.Cu) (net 13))
 (segment (start 158.54 104.429) (end 158.54 102.01) (width 0.25) (layer F.Cu) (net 14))
 (segment (start 160.4737 104.9543) (end 158.54 104.9543) (width 0.25) (layer F.Cu) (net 14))
 (segment (start 160.7904 105.271) (end 160.4737 104.9543) (width 0.25) (layer F.Cu) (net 14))
 (segment (start 160.7904 106.0659) (end 160.7904 105.271) (width 0.25) (layer F.Cu) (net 14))
 (segment (start 158.8756 107.9807) (end 160.7904 106.0659) (width 0.25) (layer F.Cu) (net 14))
 (segment (start 158.75 107.9807) (end 158.8756 107.9807) (width 0.25) (layer F.Cu) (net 14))
 (segment (start 158.75 109.156) (end 158.75 107.9807) (width 0.25) (layer F.Cu) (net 14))
 (segment (start 158.54 104.429) (end 158.54 104.9543) (width 0.25) (layer F.Cu) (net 14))
 (via (at 157.74 103.7244) (size 0.6) (layers F.Cu B.Cu) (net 11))
 (segment (start 156.21 105.2544) (end 157.74 103.7244) (width 0.25) (layer B.Cu) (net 11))
 (segment (start 156.21 109.156) (end 156.21 105.2544) (width 0.25) (layer B.Cu) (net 11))
 (segment (start 157.74 104.429) (end 157.74 103.7244) (width 0.25) (layer F.Cu) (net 11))
 (segment (start 157.74 103.7244) (end 157.74 102.01) (width 0.25) (layer F.Cu) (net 11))
 (segment (start 156.14 104.429) (end 156.4652 104.429) (width 0.25) (layer F.Cu) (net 15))
 (segment (start 156.7903 104.1039) (end 156.7903 102.01) (width 0.25) (layer F.Cu) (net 15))
 (segment (start 156.4652 104.429) (end 156.7903 104.1039) (width 0.25) (layer F.Cu) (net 15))
 (segment (start 156.14 102.01) (end 156.7903 102.01) (width 0.25) (layer F.Cu) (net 15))
 (segment (start 156.7904 104.7542) (end 156.4652 104.429) (width 0.25) (layer F.Cu) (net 15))
 (segment (start 156.7904 106.0356) (end 156.7904 104.7542) (width 0.25) (layer F.Cu) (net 15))
 (segment (start 154.8453 107.9807) (end 156.7904 106.0356) (width 0.25) (layer F.Cu) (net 15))
 (segment (start 153.67 107.9807) (end 154.8453 107.9807) (width 0.25) (layer F.Cu) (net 15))
 (segment (start 153.67 109.156) (end 153.67 107.9807) (width 0.25) (layer F.Cu) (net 15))
 (segment (start 155.34 104.429) (end 155.34 102.01) (width 0.25) (layer F.Cu) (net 16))
 (segment (start 153.3784 104.9543) (end 155.34 104.9543) (width 0.25) (layer F.Cu) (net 16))
 (segment (start 151.13 107.2027) (end 153.3784 104.9543) (width 0.25) (layer F.Cu) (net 16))
 (segment (start 151.13 109.156) (end 151.13 107.2027) (width 0.25) (layer F.Cu) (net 16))
 (segment (start 155.34 104.429) (end 155.34 104.9543) (width 0.25) (layer F.Cu) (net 16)))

